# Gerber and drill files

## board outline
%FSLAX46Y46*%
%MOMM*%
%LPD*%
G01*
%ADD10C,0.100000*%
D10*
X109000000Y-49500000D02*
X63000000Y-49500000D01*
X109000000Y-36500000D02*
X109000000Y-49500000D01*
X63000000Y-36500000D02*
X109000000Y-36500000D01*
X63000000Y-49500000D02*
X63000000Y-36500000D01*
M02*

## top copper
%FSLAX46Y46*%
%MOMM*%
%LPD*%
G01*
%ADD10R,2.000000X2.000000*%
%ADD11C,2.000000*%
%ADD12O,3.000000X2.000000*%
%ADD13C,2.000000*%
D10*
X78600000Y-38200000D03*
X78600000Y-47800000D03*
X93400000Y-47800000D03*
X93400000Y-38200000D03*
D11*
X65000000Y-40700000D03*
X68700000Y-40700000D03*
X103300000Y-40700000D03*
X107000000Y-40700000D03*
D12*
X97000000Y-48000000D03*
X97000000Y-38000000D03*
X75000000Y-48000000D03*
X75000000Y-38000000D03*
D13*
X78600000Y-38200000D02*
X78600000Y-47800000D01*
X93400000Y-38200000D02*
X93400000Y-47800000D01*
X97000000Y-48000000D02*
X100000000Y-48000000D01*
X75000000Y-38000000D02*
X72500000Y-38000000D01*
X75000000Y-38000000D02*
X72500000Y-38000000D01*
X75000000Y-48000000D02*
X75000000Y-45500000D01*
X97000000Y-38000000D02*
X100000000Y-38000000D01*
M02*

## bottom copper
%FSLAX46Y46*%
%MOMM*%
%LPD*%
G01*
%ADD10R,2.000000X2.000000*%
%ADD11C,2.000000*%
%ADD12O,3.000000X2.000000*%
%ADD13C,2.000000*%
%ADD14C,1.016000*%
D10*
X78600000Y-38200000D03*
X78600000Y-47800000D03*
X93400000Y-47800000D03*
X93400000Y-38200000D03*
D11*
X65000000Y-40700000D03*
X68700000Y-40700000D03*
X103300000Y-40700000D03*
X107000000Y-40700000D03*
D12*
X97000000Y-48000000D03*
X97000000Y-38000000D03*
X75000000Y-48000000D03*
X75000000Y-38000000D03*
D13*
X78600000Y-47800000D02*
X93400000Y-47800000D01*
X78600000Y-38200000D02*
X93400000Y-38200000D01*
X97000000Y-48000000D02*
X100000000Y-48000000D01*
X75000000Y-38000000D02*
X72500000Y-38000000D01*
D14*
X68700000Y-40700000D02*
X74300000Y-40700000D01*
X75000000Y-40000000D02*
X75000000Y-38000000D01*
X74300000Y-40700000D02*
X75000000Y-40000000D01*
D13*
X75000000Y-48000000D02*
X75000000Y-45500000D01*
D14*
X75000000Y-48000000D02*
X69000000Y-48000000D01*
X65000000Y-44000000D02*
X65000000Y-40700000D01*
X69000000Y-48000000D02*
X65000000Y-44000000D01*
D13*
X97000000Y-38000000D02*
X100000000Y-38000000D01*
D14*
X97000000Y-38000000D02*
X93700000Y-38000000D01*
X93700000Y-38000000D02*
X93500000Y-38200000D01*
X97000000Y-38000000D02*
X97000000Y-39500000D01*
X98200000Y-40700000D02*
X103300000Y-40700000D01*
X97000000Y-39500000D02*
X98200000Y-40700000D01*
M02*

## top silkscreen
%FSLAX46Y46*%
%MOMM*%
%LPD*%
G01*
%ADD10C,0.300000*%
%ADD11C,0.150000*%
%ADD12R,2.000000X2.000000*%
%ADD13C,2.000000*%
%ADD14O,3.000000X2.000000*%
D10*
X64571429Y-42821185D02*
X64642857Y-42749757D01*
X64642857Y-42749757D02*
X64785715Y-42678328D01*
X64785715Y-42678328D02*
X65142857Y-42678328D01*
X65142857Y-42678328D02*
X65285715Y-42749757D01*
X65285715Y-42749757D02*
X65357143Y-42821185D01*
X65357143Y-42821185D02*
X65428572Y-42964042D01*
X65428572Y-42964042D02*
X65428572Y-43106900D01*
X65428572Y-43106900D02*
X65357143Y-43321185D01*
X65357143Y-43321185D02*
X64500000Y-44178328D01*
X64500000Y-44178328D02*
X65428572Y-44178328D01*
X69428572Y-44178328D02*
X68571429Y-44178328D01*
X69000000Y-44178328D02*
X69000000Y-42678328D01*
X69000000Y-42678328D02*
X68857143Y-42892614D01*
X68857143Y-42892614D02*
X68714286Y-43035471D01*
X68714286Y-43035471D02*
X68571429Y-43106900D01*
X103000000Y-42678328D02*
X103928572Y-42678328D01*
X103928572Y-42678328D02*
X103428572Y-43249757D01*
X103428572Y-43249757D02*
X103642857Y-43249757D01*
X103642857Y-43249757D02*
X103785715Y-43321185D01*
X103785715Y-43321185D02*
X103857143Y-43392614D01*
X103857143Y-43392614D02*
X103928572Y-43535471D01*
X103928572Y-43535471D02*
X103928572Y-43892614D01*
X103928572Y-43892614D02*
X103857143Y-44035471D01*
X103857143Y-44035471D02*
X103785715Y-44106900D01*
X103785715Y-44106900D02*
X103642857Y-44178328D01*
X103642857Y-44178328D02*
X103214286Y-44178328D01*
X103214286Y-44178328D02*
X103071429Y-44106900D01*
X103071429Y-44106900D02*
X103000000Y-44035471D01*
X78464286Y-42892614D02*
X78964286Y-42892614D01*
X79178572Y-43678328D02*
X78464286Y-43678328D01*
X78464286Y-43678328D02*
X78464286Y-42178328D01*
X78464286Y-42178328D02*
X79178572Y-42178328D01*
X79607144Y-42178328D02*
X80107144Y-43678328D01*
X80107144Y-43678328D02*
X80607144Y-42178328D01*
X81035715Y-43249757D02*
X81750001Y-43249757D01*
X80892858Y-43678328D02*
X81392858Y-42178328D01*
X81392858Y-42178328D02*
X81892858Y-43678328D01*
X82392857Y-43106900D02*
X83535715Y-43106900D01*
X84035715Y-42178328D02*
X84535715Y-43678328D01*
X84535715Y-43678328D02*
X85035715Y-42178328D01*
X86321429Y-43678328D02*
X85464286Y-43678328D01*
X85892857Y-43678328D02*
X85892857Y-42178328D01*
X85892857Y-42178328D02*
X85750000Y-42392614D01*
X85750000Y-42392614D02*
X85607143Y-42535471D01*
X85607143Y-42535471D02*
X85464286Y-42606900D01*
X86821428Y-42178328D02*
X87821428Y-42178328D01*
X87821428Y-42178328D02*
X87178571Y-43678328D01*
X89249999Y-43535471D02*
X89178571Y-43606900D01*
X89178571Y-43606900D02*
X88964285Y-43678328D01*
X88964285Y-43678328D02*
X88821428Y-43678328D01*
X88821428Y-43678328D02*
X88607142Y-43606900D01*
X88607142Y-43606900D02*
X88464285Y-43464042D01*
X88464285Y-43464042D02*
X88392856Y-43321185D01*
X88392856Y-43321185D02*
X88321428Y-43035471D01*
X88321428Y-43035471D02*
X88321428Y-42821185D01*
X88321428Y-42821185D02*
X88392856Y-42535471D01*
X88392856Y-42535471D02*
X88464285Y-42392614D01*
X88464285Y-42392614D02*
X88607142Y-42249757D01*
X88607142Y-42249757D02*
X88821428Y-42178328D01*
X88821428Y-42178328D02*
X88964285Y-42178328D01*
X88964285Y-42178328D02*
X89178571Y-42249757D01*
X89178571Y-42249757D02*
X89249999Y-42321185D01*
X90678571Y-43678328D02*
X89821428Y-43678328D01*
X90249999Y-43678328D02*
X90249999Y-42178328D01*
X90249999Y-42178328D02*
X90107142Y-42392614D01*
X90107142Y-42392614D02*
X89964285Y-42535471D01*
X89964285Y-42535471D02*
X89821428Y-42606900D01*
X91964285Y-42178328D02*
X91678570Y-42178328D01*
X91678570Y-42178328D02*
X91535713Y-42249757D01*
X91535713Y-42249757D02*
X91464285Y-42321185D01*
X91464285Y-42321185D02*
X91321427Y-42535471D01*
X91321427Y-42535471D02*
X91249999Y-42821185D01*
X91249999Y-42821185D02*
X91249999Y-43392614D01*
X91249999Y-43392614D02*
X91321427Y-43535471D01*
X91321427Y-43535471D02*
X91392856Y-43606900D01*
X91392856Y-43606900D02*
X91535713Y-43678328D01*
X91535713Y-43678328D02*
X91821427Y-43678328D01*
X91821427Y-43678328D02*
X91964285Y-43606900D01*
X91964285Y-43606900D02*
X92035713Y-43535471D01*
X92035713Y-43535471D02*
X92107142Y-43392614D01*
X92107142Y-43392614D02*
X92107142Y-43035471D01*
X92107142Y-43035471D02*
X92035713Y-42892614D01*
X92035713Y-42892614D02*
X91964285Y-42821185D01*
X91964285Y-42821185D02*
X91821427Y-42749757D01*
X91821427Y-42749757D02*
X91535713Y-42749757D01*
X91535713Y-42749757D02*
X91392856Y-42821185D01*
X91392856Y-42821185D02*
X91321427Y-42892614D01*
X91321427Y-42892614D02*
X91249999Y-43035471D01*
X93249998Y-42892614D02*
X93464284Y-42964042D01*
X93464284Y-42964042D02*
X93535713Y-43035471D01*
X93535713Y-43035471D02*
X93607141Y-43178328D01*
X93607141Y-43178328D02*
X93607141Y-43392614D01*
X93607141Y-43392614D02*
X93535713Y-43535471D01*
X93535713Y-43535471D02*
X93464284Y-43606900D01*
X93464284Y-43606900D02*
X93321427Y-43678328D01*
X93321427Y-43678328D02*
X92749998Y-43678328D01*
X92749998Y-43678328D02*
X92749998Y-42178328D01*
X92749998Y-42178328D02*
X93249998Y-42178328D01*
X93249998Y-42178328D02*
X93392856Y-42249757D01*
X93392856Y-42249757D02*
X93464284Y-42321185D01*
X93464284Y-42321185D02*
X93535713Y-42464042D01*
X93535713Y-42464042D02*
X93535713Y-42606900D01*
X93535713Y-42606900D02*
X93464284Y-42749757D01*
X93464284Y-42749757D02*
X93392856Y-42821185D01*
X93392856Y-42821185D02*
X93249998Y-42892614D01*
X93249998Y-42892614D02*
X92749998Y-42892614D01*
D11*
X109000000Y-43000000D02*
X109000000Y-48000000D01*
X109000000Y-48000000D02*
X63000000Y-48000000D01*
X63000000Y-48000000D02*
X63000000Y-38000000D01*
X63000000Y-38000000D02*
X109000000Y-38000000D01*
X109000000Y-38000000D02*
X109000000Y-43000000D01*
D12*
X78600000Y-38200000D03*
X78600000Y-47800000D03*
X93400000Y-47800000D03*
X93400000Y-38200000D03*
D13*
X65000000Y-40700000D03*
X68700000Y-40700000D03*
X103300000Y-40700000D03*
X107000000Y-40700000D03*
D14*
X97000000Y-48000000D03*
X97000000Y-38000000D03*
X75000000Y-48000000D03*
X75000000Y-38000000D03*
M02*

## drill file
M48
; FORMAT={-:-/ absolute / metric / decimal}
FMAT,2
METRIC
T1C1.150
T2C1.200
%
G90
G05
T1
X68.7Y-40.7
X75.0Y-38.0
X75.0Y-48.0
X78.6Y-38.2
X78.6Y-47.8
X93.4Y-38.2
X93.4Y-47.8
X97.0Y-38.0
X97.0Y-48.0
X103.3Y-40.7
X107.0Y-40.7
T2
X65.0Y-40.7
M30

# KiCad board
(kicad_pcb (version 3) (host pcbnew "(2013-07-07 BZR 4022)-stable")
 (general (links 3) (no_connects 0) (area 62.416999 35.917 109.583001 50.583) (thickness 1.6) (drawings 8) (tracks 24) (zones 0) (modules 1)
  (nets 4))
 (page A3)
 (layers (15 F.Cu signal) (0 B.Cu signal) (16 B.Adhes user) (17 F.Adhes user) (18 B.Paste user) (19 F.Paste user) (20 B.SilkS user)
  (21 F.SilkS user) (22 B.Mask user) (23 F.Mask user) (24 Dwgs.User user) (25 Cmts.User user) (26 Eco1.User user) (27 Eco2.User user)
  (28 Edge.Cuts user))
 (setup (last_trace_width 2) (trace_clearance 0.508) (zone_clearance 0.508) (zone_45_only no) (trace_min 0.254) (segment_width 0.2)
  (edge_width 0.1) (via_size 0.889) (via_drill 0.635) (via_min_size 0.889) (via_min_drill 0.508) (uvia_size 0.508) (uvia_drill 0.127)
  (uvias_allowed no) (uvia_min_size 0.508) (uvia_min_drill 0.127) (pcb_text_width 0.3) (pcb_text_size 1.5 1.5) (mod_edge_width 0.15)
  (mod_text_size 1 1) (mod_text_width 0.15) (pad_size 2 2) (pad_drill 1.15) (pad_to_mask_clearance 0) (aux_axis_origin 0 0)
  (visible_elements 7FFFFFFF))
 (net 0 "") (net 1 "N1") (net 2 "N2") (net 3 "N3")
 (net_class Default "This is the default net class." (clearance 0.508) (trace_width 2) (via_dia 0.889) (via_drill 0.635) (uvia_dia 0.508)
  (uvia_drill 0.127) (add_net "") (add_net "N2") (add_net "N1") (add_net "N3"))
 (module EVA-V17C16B (layer F.Cu) (at 86 43 180)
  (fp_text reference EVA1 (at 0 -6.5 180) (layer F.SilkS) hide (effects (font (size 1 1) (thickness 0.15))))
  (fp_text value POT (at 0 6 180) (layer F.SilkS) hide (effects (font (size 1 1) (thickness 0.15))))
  (fp_line (start -23 0) (end -23 -5) (layer F.SilkS) (width 0.15))
  (fp_line (start -23 -5) (end 23 -5) (layer F.SilkS) (width 0.15))
  (fp_line (start 23 -5) (end 23 5) (layer F.SilkS) (width 0.15))
  (fp_line (start 23 5) (end -23 5) (layer F.SilkS) (width 0.15))
  (fp_line (start -23 5) (end -23 0) (layer F.SilkS) (width 0.15))
  (pad 4 thru_hole rect (at 7.4 4.8 180) (size 2 2) (drill 1.15) (layers *.Cu *.Mask F.SilkS))
  (pad 5 thru_hole rect (at 7.4 -4.8 180) (size 2 2) (drill 1.15) (layers *.Cu *.Mask F.SilkS))
  (pad 6 thru_hole rect (at -7.4 -4.8 180) (size 2 2) (drill 1.15) (layers *.Cu *.Mask F.SilkS))
  (pad 7 thru_hole rect (at -7.4 4.8 180) (size 2 2) (drill 1.15) (layers *.Cu *.Mask F.SilkS))
  (pad 2 thru_hole circle (at 21 2.3 180) (size 2 2) (drill 1.2) (layers *.Cu *.Mask F.SilkS) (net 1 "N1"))
  (pad 1 thru_hole circle (at 17.3 2.3 180) (size 2 2) (drill 1.15) (layers *.Cu *.Mask F.SilkS) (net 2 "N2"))
  (pad 3 thru_hole circle (at -17.3 2.3 180) (size 2 2) (drill 1.15) (layers *.Cu *.Mask F.SilkS) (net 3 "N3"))
  (pad 8 thru_hole circle (at -21 2.3 180) (size 2 2) (drill 1.15) (layers *.Cu *.Mask F.SilkS))
  (pad 9 thru_hole oval (at -11 -5 180) (size 3 2) (drill 1.15) (layers *.Cu *.Mask F.SilkS))
  (pad 3 thru_hole oval (at -11 5 180) (size 3 2) (drill 1.15) (layers *.Cu *.Mask F.SilkS) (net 3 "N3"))
  (pad 2 thru_hole oval (at 11 -5 180) (size 3 2) (drill 1.15) (layers *.Cu *.Mask F.SilkS) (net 1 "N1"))
  (pad 1 thru_hole oval (at 11 5 180) (size 3 2) (drill 1.15) (layers *.Cu *.Mask F.SilkS) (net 2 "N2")))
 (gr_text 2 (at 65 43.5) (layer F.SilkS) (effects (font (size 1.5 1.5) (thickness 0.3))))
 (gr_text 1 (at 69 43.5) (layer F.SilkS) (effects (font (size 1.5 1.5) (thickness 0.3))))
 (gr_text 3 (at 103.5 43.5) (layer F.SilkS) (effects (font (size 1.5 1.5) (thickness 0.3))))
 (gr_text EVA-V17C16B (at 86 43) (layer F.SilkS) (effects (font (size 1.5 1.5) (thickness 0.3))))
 (gr_line (start 109 49.5) (end 63 49.5) (angle 90) (layer Edge.Cuts) (width 0.1))
 (gr_line (start 109 36.5) (end 109 49.5) (angle 90) (layer Edge.Cuts) (width 0.1))
 (gr_line (start 63 36.5) (end 109 36.5) (angle 90) (layer Edge.Cuts) (width 0.1))
 (gr_line (start 63 49.5) (end 63 36.5) (angle 90) (layer Edge.Cuts) (width 0.1))
 (segment (start 78.6 47.8) (end 93.4 47.8) (width 2) (layer B.Cu) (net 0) (status C00000))
 (segment (start 78.6 38.2) (end 93.4 38.2) (width 2) (layer B.Cu) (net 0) (status C00000))
 (segment (start 78.6 38.2) (end 78.6 47.8) (width 2) (layer F.Cu) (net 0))
 (segment (start 93.4 38.2) (end 93.4 47.8) (width 2) (layer F.Cu) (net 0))
 (segment (start 97 48) (end 100 48) (width 2) (layer F.Cu) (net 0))
 (segment (start 97 48) (end 100 48) (width 2) (layer B.Cu) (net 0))
 (segment (start 75 38) (end 72.5 38) (width 2) (layer F.Cu) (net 2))
 (segment (start 75 38) (end 72.5 38) (width 2) (layer F.Cu) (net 2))
 (segment (start 75 38) (end 72.5 38) (width 2) (layer B.Cu) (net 2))
 (segment (start 68.7 40.7) (end 74.3 40.7) (width 1.016) (layer B.Cu) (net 2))
 (segment (start 75 40) (end 75 38) (width 1.016) (layer B.Cu) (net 2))
 (segment (start 74.3 40.7) (end 75 40) (width 1.016) (layer B.Cu) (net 2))
 (segment (start 75 48) (end 75 45.5) (width 2) (layer F.Cu) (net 1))
 (segment (start 75 48) (end 75 45.5) (width 2) (layer B.Cu) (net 1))
 (segment (start 75 48) (end 69 48) (width 1.016) (layer B.Cu) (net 1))
 (segment (start 65 44) (end 65 40.7) (width 1.016) (layer B.Cu) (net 1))
 (segment (start 69 48) (end 65 44) (width 1.016) (layer B.Cu) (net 1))
 (segment (start 97 38) (end 100 38) (width 2) (layer F.Cu) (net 3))
 (segment (start 97 38) (end 100 38) (width 2) (layer B.Cu) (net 3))
 (segment (start 97 38) (end 93.7 38) (width 1.016) (layer B.Cu) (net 3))
 (segment (start 93.7 38) (end 93.5 38.2) (width 1.016) (layer B.Cu) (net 3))
 (segment (start 97 38) (end 97 39.5) (width 1.016) (layer B.Cu) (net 3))
 (segment (start 98.2 40.7) (end 103.3 40.7) (width 1.016) (layer B.Cu) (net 3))
 (segment (start 97 39.5) (end 98.2 40.7) (width 1.016) (layer B.Cu) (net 3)))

